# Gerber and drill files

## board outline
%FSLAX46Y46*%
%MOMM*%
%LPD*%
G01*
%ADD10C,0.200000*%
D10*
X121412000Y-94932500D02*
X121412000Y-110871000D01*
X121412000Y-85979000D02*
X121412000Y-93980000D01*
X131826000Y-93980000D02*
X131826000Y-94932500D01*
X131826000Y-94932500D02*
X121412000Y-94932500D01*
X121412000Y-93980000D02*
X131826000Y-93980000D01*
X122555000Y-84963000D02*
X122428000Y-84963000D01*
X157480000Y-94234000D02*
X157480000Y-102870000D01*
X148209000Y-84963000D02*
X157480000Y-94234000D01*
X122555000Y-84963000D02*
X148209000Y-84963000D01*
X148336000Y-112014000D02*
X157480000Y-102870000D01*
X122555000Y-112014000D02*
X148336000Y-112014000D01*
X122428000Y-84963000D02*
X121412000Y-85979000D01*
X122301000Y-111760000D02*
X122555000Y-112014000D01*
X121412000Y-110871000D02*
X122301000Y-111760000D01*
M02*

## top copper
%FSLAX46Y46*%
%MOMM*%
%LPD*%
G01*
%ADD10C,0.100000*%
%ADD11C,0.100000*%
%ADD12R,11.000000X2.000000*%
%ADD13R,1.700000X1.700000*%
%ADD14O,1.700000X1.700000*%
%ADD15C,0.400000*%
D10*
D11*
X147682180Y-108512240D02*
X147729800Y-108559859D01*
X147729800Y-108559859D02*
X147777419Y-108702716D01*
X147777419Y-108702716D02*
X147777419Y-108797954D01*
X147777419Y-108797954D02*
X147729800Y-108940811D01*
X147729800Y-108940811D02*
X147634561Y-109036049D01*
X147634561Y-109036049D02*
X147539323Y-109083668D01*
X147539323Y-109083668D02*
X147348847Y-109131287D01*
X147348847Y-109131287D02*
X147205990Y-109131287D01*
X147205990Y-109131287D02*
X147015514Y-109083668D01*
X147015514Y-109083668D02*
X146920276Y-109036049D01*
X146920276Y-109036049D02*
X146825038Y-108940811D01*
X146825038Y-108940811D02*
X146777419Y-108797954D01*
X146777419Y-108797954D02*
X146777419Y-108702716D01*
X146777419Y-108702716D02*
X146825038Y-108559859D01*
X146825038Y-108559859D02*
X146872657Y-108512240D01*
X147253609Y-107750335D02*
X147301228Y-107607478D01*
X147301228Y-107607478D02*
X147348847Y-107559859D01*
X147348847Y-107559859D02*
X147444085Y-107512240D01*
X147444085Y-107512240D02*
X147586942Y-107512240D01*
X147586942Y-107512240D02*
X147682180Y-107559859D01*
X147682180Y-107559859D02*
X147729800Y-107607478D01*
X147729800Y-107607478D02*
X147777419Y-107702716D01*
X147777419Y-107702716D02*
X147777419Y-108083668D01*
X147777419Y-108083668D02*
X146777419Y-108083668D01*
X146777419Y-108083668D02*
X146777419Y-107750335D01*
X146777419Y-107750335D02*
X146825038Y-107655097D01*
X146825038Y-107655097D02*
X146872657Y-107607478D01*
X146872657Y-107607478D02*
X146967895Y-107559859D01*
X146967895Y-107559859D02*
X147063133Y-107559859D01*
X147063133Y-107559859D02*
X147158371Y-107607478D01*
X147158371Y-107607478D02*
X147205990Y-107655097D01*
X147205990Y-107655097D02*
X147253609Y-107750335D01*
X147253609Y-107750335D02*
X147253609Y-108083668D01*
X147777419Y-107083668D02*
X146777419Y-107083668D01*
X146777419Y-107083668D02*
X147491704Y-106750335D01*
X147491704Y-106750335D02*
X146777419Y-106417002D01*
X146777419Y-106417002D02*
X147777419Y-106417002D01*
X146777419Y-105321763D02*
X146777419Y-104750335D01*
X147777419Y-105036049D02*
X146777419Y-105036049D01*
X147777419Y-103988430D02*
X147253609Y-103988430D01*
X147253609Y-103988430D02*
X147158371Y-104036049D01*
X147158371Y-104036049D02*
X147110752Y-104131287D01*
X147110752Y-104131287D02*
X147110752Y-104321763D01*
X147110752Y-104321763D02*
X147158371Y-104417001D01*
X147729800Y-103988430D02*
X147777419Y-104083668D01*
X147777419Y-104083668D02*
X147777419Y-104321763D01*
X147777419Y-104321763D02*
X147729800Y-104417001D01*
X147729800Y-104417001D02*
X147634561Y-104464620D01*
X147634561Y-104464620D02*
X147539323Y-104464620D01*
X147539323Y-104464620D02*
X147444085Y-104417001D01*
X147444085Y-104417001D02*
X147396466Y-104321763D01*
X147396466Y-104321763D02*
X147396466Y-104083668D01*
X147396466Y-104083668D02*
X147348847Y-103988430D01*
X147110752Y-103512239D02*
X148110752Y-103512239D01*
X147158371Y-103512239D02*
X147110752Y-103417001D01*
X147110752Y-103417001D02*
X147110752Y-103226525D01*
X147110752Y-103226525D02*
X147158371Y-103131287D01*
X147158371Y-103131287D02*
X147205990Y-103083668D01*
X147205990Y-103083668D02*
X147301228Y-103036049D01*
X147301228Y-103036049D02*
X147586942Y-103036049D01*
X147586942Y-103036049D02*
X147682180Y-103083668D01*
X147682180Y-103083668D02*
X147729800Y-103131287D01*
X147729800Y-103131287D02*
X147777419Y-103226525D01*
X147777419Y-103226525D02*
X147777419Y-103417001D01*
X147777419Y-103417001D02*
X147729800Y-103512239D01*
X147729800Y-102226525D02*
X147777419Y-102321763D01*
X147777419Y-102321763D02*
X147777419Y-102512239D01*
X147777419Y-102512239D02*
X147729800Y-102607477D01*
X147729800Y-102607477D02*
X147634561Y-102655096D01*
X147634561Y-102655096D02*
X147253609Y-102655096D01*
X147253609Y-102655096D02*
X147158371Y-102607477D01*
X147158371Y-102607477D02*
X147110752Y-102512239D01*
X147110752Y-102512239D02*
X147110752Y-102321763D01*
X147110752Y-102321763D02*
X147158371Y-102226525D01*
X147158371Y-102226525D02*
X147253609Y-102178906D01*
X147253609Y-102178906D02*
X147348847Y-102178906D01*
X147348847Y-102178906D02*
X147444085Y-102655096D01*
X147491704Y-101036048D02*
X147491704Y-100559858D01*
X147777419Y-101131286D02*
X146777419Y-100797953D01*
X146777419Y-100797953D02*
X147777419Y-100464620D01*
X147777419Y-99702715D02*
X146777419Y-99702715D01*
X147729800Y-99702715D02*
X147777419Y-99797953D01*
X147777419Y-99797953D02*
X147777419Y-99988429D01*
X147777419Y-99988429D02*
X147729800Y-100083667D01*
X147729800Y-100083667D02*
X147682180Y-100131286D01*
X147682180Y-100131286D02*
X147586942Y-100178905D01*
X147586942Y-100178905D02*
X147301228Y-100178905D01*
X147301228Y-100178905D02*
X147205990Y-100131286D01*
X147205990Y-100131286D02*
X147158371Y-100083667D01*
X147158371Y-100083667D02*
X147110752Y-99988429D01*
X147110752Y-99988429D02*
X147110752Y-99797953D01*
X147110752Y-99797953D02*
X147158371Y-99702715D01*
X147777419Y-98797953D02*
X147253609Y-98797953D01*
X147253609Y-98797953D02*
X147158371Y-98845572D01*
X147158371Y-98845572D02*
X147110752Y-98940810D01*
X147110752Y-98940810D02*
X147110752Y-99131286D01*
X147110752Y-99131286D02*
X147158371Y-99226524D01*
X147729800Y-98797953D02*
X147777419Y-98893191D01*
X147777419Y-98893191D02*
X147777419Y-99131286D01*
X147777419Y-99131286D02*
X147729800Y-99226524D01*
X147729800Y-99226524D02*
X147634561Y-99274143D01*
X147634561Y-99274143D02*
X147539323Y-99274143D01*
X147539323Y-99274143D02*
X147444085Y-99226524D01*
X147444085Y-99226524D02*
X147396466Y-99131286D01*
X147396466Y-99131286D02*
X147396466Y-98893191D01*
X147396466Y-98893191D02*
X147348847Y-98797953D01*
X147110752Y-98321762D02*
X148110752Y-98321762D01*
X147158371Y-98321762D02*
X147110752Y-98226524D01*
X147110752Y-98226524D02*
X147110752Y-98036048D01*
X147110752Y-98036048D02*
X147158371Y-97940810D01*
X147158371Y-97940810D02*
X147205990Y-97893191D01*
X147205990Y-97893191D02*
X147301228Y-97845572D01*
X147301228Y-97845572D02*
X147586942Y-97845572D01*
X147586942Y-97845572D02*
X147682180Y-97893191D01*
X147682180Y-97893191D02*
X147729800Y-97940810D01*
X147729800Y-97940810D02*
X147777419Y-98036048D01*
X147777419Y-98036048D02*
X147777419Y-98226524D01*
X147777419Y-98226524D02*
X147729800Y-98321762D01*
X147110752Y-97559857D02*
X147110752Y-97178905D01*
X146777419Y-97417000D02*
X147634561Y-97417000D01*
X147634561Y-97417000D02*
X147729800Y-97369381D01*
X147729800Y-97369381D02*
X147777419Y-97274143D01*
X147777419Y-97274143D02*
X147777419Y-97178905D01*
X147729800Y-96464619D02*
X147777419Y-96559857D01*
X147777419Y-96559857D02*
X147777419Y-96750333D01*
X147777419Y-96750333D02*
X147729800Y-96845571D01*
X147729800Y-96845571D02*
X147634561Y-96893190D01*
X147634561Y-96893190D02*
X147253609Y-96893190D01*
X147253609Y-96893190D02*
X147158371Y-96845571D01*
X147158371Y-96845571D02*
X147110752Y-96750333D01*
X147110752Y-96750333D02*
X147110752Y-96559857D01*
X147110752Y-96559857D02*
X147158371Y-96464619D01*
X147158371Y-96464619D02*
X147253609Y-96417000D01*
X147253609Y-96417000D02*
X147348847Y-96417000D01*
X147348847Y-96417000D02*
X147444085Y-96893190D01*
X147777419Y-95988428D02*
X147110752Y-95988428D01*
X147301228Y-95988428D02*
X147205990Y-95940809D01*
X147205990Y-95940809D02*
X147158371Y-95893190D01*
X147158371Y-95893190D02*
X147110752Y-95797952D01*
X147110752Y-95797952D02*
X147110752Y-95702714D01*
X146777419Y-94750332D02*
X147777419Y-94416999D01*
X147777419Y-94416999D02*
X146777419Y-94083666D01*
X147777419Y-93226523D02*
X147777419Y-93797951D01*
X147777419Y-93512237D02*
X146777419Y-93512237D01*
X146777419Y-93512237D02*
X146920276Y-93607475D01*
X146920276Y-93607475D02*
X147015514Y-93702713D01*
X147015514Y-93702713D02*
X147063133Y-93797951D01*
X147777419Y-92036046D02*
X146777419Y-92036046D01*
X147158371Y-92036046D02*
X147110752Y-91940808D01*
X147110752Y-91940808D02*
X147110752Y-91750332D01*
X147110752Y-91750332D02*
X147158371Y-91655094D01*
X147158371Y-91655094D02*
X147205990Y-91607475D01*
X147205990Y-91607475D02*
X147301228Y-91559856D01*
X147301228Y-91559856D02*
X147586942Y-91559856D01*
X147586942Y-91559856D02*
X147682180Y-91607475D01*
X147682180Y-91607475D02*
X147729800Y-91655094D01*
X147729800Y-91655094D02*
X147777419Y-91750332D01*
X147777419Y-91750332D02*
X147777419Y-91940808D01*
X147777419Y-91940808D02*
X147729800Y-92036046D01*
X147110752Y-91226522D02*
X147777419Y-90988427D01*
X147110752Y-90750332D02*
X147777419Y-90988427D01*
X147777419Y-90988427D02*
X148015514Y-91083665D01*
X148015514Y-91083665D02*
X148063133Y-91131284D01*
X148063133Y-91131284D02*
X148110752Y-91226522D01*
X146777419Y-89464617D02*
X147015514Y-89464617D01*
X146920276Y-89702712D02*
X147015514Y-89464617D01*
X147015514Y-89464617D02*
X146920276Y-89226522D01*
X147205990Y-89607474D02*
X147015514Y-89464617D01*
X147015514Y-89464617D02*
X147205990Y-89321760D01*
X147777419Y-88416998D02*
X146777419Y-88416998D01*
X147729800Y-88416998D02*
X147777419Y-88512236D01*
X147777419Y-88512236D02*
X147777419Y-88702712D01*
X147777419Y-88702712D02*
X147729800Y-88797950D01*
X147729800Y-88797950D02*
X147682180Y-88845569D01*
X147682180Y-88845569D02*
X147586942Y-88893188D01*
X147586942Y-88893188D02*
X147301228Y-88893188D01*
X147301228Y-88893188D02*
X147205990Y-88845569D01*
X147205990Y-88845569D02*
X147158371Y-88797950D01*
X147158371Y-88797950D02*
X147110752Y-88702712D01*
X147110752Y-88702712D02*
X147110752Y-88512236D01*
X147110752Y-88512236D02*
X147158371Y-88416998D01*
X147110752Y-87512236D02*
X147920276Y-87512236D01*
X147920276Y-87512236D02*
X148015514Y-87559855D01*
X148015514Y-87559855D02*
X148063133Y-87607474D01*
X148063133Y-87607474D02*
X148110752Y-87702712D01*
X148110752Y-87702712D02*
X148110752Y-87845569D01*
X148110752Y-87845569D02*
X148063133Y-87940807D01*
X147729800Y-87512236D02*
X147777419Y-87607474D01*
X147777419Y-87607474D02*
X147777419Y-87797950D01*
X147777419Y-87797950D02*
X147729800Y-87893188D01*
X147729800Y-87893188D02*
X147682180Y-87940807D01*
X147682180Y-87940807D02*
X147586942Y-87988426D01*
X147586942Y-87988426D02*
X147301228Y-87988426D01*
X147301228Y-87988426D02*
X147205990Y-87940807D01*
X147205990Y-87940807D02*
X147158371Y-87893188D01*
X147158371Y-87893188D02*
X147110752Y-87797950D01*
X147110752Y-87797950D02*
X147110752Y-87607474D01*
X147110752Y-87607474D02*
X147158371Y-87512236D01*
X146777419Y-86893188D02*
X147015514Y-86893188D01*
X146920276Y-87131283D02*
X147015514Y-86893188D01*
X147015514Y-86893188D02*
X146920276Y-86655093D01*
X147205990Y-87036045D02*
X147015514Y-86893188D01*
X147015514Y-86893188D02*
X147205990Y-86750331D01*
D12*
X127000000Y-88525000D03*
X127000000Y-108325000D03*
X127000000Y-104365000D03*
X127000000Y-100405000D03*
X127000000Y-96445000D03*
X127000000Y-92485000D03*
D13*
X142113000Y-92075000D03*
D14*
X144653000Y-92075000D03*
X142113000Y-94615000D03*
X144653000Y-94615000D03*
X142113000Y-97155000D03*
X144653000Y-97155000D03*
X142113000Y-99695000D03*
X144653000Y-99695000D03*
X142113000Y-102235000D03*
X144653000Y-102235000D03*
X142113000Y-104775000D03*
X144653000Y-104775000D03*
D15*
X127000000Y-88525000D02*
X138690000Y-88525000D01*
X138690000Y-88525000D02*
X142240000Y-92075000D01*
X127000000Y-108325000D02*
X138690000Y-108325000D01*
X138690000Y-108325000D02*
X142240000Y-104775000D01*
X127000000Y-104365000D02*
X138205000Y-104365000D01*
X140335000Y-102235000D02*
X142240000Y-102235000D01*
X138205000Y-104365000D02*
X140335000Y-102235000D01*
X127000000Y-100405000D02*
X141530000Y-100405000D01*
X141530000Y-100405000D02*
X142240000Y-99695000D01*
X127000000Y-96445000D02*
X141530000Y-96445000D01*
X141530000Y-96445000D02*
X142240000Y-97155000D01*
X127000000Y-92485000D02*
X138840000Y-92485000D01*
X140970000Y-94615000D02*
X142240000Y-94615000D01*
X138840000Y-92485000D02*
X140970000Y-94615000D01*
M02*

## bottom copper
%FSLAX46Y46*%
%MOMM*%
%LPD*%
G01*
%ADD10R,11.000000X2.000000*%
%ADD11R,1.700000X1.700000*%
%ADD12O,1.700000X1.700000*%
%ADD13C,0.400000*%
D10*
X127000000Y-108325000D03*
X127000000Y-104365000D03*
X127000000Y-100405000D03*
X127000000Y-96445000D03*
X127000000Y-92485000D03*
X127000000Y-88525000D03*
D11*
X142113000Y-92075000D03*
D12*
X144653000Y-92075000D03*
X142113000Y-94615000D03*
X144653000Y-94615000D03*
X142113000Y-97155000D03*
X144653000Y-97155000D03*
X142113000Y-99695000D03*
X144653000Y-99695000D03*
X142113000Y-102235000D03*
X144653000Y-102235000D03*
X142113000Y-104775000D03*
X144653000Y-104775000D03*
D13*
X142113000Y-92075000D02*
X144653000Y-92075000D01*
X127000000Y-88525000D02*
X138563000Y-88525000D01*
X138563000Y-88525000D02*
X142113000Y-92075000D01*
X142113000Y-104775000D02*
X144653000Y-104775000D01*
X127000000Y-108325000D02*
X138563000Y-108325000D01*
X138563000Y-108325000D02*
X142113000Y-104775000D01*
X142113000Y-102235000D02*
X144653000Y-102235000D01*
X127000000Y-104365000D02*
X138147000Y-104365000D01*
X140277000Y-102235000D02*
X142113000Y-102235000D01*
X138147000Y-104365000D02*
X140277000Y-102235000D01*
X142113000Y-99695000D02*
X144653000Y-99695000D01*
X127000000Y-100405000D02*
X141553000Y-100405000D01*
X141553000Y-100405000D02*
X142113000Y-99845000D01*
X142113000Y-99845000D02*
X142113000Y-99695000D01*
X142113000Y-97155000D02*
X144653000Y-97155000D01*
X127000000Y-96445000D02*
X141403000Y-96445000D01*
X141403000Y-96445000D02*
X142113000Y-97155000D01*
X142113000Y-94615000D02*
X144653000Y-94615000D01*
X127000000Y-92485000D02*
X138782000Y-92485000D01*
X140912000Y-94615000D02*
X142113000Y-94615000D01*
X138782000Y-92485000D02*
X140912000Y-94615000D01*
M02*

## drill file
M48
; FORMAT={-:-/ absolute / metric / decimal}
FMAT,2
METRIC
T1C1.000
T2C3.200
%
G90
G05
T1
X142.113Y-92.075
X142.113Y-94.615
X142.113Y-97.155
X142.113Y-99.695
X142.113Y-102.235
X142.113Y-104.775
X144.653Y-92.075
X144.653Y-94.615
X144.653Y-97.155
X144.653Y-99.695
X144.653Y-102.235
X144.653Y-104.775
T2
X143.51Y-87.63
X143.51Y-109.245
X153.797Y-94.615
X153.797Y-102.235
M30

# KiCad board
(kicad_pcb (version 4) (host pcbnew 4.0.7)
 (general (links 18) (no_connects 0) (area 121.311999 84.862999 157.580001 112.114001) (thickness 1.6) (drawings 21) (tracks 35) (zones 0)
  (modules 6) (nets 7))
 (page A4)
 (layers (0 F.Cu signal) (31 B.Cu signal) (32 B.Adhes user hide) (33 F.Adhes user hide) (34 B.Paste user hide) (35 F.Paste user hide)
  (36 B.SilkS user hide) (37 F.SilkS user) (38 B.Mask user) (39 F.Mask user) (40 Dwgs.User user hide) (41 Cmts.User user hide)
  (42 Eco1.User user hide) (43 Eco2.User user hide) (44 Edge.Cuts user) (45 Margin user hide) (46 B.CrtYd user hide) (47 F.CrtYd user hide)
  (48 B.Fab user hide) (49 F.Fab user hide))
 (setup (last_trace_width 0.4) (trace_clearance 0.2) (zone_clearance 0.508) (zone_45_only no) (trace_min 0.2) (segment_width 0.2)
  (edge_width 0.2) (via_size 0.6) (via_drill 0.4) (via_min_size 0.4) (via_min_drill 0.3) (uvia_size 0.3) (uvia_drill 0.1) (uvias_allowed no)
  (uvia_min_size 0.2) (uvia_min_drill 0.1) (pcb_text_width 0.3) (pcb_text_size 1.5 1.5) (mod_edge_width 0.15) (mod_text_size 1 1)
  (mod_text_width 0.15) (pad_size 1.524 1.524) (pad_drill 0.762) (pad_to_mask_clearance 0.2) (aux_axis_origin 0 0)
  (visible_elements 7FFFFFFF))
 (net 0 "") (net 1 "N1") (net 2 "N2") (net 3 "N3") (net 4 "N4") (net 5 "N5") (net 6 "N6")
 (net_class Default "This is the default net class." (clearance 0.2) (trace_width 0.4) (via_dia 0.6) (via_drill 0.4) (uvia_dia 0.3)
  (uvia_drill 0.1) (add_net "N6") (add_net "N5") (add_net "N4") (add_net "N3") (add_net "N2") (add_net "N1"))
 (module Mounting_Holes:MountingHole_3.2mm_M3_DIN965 (layer F.Cu) (at 143.51 87.63)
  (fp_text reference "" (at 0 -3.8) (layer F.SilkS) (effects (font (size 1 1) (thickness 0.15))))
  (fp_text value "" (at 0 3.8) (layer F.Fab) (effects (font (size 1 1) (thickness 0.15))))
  (pad 1 np_thru_hole circle (at 0 0) (size 3.2 3.2) (drill 3.2) (layers *.Cu *.Mask)))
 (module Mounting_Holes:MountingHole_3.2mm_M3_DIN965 (layer F.Cu) (at 143.51 109.2454)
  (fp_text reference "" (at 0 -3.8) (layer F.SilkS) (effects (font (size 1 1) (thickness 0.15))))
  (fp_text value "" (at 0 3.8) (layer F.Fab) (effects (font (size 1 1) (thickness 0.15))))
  (pad 1 np_thru_hole circle (at 0 0) (size 3.2 3.2) (drill 3.2) (layers *.Cu *.Mask)))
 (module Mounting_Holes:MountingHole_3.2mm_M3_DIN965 (layer F.Cu) (at 153.797 94.615)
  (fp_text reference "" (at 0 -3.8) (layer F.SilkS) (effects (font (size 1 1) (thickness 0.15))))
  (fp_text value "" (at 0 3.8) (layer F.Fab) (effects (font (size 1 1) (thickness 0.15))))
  (pad 1 np_thru_hole circle (at 0 0) (size 3.2 3.2) (drill 3.2) (layers *.Cu *.Mask)))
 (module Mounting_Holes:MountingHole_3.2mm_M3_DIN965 (layer F.Cu) (at 153.797 102.235)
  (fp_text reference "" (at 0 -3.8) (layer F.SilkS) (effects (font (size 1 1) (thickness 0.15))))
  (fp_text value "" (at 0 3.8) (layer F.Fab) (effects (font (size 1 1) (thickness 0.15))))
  (pad 1 np_thru_hole circle (at 0 0) (size 3.2 3.2) (drill 3.2) (layers *.Cu *.Mask)))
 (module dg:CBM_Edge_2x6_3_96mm (layer F.Cu) (at 127 98.425)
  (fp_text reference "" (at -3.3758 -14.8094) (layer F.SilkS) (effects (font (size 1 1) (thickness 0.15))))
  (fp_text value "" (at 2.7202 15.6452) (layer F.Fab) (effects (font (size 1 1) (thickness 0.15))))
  (pad F connect rect (at 0 9.9) (size 11 2) (layers B.Cu B.Mask) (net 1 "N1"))
  (pad E connect rect (at 0 5.94) (size 11 2) (layers B.Cu B.Mask) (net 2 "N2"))
  (pad D connect rect (at 0 1.98) (size 11 2) (layers B.Cu B.Mask) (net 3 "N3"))
  (pad C connect rect (at 0 -1.98) (size 11 2) (layers B.Cu B.Mask) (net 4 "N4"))
  (pad B connect rect (at 0 -5.94) (size 11 2) (layers *.Mask B.Cu) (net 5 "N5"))
  (pad A connect rect (at 0 -9.9) (size 11 2) (layers *.Mask B.Cu) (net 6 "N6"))
  (pad 1 connect rect (at 0 -9.9) (size 11 2) (layers F.Cu F.Mask) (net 6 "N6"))
  (pad 6 connect rect (at 0 9.9) (size 11 2) (layers F.Cu F.Mask) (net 1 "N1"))
  (pad 5 connect rect (at 0 5.94) (size 11 2) (layers F.Cu F.Mask) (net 2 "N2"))
  (pad 4 connect rect (at 0 1.98) (size 11 2) (layers F.Cu F.Mask) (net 3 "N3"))
  (pad 3 connect rect (at 0 -1.98) (size 11 2) (layers F.Cu F.Mask) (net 4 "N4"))
  (pad 2 connect rect (at 0 -5.94) (size 11 2) (layers F.Cu F.Mask) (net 5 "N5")))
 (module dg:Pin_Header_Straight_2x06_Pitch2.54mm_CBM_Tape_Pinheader (layer F.Cu) (at 142.113 92.075)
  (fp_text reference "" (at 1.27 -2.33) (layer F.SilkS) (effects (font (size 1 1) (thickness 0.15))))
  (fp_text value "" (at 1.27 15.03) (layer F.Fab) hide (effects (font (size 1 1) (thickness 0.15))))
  (pad 1 thru_hole rect (at 0 0) (size 1.7 1.7) (drill 1) (layers *.Cu *.Mask) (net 6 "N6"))
  (pad A thru_hole oval (at 2.54 0) (size 1.7 1.7) (drill 1) (layers *.Cu *.Mask) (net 6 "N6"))
  (pad 2 thru_hole oval (at 0 2.54) (size 1.7 1.7) (drill 1) (layers *.Cu *.Mask) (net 5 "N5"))
  (pad B thru_hole oval (at 2.54 2.54) (size 1.7 1.7) (drill 1) (layers *.Cu *.Mask) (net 5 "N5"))
  (pad 3 thru_hole oval (at 0 5.08) (size 1.7 1.7) (drill 1) (layers *.Cu *.Mask) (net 4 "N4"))
  (pad C thru_hole oval (at 2.54 5.08) (size 1.7 1.7) (drill 1) (layers *.Cu *.Mask) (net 4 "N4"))
  (pad 4 thru_hole oval (at 0 7.62) (size 1.7 1.7) (drill 1) (layers *.Cu *.Mask) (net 3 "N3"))
  (pad D thru_hole oval (at 2.54 7.62) (size 1.7 1.7) (drill 1) (layers *.Cu *.Mask) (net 3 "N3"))
  (pad 5 thru_hole oval (at 0 10.16) (size 1.7 1.7) (drill 1) (layers *.Cu *.Mask) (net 2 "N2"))
  (pad E thru_hole oval (at 2.54 10.16) (size 1.7 1.7) (drill 1) (layers *.Cu *.Mask) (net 2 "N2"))
  (pad 6 thru_hole oval (at 0 12.7) (size 1.7 1.7) (drill 1) (layers *.Cu *.Mask) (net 1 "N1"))
  (pad F thru_hole oval (at 2.54 12.7) (size 1.7 1.7) (drill 1) (layers *.Cu *.Mask) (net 1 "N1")))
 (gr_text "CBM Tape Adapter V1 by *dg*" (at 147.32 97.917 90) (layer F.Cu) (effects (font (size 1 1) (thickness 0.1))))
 (gr_line (start 121.412 94.9325) (end 121.412 110.871) (angle 90) (layer Edge.Cuts) (width 0.2))
 (gr_line (start 121.412 85.979) (end 121.412 93.98) (angle 90) (layer Edge.Cuts) (width 0.2))
 (gr_line (start 131.826 93.98) (end 131.826 94.9325) (angle 90) (layer Edge.Cuts) (width 0.2))
 (gr_line (start 131.826 94.9325) (end 121.412 94.9325) (angle 90) (layer Edge.Cuts) (width 0.2))
 (gr_line (start 121.412 93.98) (end 131.826 93.98) (angle 90) (layer Edge.Cuts) (width 0.2))
 (gr_line (start 122.555 84.963) (end 122.428 84.963) (angle 90) (layer Edge.Cuts) (width 0.2))
 (gr_line (start 157.48 94.234) (end 157.48 102.87) (angle 90) (layer Edge.Cuts) (width 0.2))
 (gr_line (start 148.209 84.963) (end 157.48 94.234) (angle 90) (layer Edge.Cuts) (width 0.2))
 (gr_line (start 122.555 84.963) (end 148.209 84.963) (angle 90) (layer Edge.Cuts) (width 0.2))
 (gr_line (start 148.336 112.014) (end 157.48 102.87) (angle 90) (layer Edge.Cuts) (width 0.2))
 (gr_line (start 122.555 112.014) (end 148.336 112.014) (angle 90) (layer Edge.Cuts) (width 0.2))
 (gr_line (start 122.428 84.963) (end 121.412 85.979) (angle 90) (layer Edge.Cuts) (width 0.2))
 (gr_line (start 122.301 111.76) (end 122.555 112.014) (angle 90) (layer Edge.Cuts) (width 0.2))
 (gr_line (start 121.412 110.871) (end 122.301 111.76) (angle 90) (layer Edge.Cuts) (width 0.2))
 (segment (start 142.113 92.075) (end 144.653 92.075) (width 0.4) (layer B.Cu) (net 6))
 (segment (start 127 88.525) (end 138.563 88.525) (width 0.4) (layer B.Cu) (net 6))
 (segment (start 138.563 88.525) (end 142.113 92.075) (width 0.4) (layer B.Cu) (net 6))
 (segment (start 127 88.525) (end 138.69 88.525) (width 0.4) (layer F.Cu) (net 6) (status 10))
 (segment (start 138.69 88.525) (end 142.24 92.075) (width 0.4) (layer F.Cu) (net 6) (status 20))
 (segment (start 142.113 104.775) (end 144.653 104.775) (width 0.4) (layer B.Cu) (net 1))
 (segment (start 127 108.325) (end 138.563 108.325) (width 0.4) (layer B.Cu) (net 1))
 (segment (start 138.563 108.325) (end 142.113 104.775) (width 0.4) (layer B.Cu) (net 1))
 (segment (start 127 108.325) (end 138.69 108.325) (width 0.4) (layer F.Cu) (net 1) (status 10))
 (segment (start 138.69 108.325) (end 142.24 104.775) (width 0.4) (layer F.Cu) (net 1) (status 20))
 (segment (start 142.113 102.235) (end 144.653 102.235) (width 0.4) (layer B.Cu) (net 2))
 (segment (start 127 104.365) (end 138.147 104.365) (width 0.4) (layer B.Cu) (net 2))
 (segment (start 140.277 102.235) (end 142.113 102.235) (width 0.4) (layer B.Cu) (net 2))
 (segment (start 138.147 104.365) (end 140.277 102.235) (width 0.4) (layer B.Cu) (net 2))
 (segment (start 127 104.365) (end 138.205 104.365) (width 0.4) (layer F.Cu) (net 2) (status 10))
 (segment (start 140.335 102.235) (end 142.24 102.235) (width 0.4) (layer F.Cu) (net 2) (status 20))
 (segment (start 138.205 104.365) (end 140.335 102.235) (width 0.4) (layer F.Cu) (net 2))
 (segment (start 142.113 99.695) (end 144.653 99.695) (width 0.4) (layer B.Cu) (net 3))
 (segment (start 127 100.405) (end 141.553 100.405) (width 0.4) (layer B.Cu) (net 3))
 (segment (start 141.553 100.405) (end 142.113 99.845) (width 0.4) (layer B.Cu) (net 3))
 (segment (start 142.113 99.845) (end 142.113 99.695) (width 0.4) (layer B.Cu) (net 3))
 (segment (start 127 100.405) (end 141.53 100.405) (width 0.4) (layer F.Cu) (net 3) (status 10))
 (segment (start 141.53 100.405) (end 142.24 99.695) (width 0.4) (layer F.Cu) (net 3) (status 20))
 (segment (start 142.113 97.155) (end 144.653 97.155) (width 0.4) (layer B.Cu) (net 4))
 (segment (start 127 96.445) (end 141.403 96.445) (width 0.4) (layer B.Cu) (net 4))
 (segment (start 141.403 96.445) (end 142.113 97.155) (width 0.4) (layer B.Cu) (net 4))
 (segment (start 127 96.445) (end 141.53 96.445) (width 0.4) (layer F.Cu) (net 4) (status 10))
 (segment (start 141.53 96.445) (end 142.24 97.155) (width 0.4) (layer F.Cu) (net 4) (status 20))
 (segment (start 142.113 94.615) (end 144.653 94.615) (width 0.4) (layer B.Cu) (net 5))
 (segment (start 127 92.485) (end 138.782 92.485) (width 0.4) (layer B.Cu) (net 5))
 (segment (start 140.912 94.615) (end 142.113 94.615) (width 0.4) (layer B.Cu) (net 5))
 (segment (start 138.782 92.485) (end 140.912 94.615) (width 0.4) (layer B.Cu) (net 5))
 (segment (start 127 92.485) (end 138.84 92.485) (width 0.4) (layer F.Cu) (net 5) (status 10))
 (segment (start 140.97 94.615) (end 142.24 94.615) (width 0.4) (layer F.Cu) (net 5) (status 20))
 (segment (start 138.84 92.485) (end 140.97 94.615) (width 0.4) (layer F.Cu) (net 5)))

